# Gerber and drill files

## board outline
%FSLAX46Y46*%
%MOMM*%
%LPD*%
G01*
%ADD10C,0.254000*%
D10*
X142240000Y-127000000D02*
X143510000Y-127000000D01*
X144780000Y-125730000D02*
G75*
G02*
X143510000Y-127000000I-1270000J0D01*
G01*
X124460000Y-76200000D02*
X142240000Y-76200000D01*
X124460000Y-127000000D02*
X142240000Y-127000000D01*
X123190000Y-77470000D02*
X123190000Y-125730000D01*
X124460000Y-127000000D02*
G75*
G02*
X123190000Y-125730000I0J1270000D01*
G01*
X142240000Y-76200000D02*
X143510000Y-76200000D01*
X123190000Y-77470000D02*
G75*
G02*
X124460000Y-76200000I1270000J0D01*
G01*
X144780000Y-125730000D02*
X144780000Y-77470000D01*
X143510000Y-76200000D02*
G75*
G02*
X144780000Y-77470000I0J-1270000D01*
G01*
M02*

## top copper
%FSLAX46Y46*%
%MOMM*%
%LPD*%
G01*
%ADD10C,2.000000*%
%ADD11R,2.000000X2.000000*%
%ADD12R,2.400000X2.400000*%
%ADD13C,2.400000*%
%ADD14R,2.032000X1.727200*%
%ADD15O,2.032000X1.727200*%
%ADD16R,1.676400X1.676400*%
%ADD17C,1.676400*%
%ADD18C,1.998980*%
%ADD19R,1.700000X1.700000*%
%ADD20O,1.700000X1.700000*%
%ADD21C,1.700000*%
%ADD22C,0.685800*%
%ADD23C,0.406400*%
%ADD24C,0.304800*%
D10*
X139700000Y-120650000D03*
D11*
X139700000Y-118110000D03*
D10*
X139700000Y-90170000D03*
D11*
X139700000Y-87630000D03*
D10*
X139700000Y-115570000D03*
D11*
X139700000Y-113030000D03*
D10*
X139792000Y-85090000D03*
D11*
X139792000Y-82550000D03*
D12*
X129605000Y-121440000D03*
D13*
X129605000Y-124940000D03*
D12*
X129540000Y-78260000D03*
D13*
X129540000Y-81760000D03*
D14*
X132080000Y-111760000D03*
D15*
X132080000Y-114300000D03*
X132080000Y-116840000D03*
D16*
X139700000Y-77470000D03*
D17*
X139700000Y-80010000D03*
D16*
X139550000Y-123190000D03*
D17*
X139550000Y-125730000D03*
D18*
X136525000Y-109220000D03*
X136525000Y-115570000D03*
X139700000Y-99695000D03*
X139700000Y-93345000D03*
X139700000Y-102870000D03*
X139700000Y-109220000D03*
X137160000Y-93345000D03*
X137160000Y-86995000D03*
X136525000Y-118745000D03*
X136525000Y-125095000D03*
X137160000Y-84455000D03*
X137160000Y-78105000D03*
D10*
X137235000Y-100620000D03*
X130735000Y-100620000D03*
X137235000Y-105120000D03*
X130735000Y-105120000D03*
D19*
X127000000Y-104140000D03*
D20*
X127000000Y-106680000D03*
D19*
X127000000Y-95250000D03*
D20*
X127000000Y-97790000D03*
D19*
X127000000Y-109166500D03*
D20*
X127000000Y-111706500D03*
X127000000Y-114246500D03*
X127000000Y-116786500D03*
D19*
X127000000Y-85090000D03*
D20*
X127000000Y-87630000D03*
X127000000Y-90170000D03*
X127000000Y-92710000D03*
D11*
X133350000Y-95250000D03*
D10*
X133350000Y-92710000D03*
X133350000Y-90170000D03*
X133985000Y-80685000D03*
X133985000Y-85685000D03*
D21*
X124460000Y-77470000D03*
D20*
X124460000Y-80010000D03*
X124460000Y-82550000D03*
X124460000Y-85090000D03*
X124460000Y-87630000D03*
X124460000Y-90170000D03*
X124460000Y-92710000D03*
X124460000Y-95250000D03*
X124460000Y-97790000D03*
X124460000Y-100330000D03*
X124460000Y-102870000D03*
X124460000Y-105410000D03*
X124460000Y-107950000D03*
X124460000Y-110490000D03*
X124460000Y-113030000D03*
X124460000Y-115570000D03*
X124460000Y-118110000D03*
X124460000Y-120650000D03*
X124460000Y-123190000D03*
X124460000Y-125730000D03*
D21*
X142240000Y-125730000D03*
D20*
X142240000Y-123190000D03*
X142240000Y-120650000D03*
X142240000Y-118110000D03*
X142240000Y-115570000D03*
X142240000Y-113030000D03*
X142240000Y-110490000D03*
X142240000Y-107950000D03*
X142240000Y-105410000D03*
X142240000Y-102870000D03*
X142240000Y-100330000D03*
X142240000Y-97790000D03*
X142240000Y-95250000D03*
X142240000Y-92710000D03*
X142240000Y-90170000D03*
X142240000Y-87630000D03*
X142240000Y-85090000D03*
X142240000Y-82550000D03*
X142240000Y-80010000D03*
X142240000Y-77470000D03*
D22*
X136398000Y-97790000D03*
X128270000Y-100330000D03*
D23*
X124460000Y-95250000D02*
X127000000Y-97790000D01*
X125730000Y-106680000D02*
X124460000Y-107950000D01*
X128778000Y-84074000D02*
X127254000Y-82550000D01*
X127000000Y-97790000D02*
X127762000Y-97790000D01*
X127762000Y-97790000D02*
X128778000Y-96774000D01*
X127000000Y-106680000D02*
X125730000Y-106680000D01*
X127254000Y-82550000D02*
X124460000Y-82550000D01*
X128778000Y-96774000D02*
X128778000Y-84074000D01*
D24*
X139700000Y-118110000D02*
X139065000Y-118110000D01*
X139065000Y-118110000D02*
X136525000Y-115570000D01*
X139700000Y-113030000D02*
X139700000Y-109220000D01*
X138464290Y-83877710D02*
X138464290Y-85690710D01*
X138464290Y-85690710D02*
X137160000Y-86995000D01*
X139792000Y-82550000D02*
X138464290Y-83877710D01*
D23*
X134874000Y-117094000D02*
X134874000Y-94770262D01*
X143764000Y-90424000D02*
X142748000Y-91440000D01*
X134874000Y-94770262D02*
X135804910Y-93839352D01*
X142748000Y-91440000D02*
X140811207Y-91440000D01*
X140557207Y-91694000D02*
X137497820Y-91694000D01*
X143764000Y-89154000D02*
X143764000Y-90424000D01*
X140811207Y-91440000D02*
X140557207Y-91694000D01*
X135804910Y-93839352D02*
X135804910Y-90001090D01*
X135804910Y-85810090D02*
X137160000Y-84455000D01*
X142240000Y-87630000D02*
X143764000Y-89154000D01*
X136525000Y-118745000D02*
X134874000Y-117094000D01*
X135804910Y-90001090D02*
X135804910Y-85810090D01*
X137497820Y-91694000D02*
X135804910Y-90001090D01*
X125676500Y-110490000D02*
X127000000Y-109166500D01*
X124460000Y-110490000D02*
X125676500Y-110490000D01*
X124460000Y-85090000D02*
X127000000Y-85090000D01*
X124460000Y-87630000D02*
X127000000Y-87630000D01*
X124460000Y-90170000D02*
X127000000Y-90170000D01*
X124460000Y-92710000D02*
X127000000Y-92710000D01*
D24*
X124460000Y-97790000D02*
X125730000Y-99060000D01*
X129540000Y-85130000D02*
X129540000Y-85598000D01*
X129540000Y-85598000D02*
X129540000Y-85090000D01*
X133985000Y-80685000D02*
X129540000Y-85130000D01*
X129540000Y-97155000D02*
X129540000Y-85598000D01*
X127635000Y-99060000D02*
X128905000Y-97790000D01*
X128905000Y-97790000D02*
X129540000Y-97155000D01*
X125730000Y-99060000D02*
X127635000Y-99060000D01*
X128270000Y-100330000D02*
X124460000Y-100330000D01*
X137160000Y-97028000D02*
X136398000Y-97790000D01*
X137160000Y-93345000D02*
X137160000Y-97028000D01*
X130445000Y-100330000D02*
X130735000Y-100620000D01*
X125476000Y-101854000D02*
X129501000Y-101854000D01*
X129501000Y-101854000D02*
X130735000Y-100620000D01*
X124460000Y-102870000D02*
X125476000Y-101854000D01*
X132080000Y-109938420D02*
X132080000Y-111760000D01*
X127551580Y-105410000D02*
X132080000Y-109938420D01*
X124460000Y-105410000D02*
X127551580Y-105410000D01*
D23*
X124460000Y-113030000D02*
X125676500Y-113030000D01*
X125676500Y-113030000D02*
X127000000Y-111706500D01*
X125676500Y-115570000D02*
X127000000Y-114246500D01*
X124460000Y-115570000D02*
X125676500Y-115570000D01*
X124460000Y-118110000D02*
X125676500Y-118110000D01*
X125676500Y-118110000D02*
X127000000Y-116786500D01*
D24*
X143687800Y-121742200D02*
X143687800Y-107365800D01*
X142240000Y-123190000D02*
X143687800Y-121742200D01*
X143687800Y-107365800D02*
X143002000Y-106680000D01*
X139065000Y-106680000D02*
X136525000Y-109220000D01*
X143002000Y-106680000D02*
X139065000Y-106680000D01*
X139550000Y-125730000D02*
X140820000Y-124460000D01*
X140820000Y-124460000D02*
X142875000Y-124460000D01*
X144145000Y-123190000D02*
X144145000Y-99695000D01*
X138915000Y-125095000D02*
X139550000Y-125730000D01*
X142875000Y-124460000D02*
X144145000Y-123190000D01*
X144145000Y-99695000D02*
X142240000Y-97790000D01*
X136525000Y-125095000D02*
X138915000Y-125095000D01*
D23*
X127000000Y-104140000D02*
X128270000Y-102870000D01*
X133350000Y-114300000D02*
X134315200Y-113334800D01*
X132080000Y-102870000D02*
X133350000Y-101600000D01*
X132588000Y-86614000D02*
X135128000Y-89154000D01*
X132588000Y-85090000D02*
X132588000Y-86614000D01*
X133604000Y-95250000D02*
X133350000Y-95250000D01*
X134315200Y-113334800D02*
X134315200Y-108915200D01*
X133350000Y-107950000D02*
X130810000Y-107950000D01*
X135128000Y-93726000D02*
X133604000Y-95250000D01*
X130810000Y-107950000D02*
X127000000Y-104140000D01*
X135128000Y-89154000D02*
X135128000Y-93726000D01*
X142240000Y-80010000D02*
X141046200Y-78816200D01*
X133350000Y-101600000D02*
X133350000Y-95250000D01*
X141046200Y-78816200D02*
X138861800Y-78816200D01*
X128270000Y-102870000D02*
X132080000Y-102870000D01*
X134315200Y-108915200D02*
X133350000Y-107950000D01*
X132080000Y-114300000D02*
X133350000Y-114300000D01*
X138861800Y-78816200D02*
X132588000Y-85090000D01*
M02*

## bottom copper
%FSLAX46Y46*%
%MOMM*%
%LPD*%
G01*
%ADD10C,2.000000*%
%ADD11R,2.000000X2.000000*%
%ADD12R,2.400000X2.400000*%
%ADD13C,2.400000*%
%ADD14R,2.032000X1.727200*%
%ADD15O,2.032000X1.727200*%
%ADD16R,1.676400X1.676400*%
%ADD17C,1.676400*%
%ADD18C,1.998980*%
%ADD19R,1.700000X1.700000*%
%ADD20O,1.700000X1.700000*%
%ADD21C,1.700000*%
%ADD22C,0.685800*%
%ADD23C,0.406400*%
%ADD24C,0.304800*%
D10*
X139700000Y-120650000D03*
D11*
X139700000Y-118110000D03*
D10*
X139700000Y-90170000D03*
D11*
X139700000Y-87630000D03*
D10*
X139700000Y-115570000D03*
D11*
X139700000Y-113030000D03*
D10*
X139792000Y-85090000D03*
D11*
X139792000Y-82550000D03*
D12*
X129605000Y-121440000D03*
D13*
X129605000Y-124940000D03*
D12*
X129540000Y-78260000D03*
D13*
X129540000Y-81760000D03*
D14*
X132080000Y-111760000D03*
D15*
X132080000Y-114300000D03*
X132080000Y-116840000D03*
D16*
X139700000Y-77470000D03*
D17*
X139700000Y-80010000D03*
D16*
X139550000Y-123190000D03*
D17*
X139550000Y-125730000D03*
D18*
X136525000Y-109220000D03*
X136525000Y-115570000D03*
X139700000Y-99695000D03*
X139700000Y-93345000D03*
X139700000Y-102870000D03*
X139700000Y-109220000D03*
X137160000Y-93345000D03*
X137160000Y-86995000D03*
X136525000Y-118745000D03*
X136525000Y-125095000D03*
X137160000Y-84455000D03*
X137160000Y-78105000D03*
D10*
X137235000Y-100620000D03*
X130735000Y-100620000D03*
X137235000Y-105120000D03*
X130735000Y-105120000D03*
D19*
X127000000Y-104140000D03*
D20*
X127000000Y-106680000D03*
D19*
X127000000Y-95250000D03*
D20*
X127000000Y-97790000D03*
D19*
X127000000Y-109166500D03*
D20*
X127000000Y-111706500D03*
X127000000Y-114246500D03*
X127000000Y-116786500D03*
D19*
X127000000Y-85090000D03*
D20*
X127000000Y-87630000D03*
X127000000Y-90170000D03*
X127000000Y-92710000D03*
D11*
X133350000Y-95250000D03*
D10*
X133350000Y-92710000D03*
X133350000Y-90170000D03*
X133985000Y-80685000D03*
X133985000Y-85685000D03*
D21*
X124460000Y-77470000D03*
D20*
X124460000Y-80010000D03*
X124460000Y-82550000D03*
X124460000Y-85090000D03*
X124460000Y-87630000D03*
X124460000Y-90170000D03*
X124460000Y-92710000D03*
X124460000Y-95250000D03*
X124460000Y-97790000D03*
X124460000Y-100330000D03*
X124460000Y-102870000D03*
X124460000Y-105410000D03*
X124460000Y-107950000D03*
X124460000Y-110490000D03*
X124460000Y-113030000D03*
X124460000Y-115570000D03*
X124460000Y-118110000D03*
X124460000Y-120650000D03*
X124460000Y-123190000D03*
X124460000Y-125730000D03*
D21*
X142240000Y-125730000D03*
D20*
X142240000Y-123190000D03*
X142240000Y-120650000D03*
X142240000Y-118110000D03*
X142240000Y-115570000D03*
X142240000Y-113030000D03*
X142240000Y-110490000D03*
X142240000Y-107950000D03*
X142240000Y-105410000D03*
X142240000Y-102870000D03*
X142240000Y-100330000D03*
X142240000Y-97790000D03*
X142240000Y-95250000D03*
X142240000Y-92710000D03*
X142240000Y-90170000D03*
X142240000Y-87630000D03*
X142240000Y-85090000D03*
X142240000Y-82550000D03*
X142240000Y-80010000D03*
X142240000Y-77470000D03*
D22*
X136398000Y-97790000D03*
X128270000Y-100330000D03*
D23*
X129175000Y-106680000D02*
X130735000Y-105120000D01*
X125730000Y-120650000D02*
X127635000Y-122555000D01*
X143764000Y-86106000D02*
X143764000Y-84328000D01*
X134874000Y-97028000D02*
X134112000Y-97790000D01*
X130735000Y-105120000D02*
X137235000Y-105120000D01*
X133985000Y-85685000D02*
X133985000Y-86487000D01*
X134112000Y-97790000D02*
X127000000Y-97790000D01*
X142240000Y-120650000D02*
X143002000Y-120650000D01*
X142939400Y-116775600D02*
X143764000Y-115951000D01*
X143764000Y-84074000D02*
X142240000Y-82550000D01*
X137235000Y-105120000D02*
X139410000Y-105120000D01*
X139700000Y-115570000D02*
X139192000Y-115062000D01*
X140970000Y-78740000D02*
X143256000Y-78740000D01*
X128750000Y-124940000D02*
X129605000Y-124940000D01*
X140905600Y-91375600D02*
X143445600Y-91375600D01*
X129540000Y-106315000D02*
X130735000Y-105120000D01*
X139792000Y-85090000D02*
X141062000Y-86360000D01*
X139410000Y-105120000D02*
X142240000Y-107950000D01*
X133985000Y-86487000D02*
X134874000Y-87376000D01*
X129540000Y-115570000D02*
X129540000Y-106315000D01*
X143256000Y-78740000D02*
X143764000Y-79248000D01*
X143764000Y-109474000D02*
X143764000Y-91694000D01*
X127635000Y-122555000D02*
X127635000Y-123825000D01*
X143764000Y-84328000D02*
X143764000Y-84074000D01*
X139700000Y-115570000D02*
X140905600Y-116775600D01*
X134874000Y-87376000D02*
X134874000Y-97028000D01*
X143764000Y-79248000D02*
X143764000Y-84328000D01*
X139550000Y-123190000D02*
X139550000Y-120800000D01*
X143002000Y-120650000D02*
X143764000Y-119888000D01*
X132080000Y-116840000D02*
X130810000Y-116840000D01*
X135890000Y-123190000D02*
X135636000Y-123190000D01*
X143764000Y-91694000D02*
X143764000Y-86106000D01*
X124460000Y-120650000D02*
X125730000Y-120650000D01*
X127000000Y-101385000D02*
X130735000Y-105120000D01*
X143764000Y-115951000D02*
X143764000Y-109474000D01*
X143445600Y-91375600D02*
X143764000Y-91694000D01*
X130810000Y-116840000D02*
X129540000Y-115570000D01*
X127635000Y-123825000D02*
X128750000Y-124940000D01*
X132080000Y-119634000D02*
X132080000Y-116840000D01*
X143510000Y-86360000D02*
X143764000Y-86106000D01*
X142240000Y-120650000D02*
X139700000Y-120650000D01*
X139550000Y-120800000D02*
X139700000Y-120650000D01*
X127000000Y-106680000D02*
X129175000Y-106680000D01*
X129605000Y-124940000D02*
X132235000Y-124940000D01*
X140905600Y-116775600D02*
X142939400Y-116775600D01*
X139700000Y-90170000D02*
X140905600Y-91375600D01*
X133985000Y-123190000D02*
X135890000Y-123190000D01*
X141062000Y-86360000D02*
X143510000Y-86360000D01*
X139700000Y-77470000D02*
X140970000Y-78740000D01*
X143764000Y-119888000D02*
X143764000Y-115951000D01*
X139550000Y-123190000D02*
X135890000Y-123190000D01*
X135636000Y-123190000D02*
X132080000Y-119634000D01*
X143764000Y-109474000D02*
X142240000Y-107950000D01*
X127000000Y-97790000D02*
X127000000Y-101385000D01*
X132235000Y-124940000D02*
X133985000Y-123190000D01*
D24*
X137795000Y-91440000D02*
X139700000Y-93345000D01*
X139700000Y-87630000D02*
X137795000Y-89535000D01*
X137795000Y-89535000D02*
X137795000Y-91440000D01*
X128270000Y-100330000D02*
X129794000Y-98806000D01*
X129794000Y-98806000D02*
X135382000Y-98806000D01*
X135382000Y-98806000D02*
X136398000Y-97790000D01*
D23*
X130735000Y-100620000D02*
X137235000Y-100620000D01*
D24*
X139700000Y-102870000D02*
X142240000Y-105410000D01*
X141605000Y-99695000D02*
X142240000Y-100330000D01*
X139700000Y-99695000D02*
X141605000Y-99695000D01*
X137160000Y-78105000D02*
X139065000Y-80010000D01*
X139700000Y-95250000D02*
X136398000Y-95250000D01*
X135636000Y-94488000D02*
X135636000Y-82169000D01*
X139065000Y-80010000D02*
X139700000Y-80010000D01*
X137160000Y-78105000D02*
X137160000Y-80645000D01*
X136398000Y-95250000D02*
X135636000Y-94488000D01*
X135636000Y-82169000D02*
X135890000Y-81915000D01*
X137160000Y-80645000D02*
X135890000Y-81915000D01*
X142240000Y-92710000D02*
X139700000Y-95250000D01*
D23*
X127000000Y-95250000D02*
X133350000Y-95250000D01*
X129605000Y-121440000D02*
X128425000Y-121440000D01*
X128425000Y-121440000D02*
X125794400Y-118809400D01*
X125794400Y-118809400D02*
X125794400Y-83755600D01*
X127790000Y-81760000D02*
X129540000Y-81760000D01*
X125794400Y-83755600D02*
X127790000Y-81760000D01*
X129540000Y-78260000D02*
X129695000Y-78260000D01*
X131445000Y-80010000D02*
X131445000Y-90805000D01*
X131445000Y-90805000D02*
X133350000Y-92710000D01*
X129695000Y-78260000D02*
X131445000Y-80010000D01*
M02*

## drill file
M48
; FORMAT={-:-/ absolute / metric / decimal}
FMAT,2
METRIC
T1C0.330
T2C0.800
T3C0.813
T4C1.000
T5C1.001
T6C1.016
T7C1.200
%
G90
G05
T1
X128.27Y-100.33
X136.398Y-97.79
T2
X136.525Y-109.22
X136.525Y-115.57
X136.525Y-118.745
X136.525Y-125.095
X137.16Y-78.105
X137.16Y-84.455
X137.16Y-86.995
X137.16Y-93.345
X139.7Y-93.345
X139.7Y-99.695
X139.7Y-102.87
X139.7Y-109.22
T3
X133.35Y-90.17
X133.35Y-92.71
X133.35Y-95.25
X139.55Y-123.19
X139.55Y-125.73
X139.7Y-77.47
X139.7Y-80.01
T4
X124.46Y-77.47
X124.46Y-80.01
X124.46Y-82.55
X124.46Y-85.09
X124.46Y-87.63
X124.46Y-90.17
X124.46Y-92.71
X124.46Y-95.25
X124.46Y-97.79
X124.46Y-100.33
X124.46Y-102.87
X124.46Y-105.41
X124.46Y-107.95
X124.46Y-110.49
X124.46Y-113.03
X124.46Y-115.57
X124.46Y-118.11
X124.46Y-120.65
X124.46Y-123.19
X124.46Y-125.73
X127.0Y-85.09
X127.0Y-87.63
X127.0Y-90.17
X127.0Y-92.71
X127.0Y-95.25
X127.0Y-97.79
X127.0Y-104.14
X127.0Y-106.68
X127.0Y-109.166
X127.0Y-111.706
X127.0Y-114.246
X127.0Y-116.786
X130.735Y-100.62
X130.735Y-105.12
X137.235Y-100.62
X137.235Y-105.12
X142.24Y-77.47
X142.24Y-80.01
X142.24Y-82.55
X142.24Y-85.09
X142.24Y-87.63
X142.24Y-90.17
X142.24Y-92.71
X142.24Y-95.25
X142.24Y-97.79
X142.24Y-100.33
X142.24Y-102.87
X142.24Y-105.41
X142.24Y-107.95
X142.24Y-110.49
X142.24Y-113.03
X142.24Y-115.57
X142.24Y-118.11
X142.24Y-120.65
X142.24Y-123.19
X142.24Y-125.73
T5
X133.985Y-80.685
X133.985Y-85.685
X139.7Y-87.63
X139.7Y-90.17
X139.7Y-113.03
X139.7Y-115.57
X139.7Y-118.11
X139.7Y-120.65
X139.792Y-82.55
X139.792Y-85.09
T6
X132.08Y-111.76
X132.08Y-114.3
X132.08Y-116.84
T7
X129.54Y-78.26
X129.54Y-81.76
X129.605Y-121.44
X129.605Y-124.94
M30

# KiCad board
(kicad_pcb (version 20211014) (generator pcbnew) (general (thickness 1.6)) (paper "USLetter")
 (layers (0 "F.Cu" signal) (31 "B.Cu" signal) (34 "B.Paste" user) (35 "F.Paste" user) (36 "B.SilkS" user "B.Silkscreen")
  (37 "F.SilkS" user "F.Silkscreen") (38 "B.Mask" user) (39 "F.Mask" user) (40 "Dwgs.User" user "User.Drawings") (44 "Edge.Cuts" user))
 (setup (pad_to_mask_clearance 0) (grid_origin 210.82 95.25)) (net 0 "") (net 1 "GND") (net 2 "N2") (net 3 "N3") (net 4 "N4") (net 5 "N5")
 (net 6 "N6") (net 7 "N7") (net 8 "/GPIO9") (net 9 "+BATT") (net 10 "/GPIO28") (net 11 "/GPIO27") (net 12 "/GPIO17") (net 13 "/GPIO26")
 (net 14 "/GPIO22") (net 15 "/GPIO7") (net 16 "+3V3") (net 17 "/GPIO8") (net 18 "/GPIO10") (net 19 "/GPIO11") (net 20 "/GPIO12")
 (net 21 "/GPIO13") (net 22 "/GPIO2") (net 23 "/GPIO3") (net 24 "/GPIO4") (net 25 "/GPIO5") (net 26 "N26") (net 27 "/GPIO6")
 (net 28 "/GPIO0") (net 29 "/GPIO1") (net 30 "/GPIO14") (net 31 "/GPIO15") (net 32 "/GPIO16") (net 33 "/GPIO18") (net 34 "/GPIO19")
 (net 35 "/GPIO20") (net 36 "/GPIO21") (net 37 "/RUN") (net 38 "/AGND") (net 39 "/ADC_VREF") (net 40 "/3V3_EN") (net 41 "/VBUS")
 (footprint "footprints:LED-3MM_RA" (layer "F.Cu") (at 139.7 120.65 90)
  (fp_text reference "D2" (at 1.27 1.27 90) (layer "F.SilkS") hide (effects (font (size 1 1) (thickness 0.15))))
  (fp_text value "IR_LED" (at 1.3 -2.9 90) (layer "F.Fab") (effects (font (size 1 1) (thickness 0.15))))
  (pad "1" thru_hole circle locked (at 0 0 180) (size 2 2) (drill 1.00076) (layers *.Cu *.Mask "F.SilkS") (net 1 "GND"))
  (pad "2" thru_hole rect locked (at 2.54 0 90) (size 2 2) (drill 1.00076) (layers *.Cu *.Mask "F.SilkS") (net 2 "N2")))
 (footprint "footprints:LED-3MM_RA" (layer "F.Cu") (at 139.7 90.17 90)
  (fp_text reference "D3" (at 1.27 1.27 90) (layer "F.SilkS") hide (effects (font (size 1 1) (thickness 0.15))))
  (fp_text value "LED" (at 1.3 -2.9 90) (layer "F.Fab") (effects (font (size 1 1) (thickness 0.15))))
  (pad "1" thru_hole circle locked (at 0 0 180) (size 2 2) (drill 1.00076) (layers *.Cu *.Mask "F.SilkS") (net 1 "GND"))
  (pad "2" thru_hole rect locked (at 2.54 0 90) (size 2 2) (drill 1.00076) (layers *.Cu *.Mask "F.SilkS") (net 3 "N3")))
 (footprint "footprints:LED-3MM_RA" (layer "F.Cu") (at 139.7 115.57 90)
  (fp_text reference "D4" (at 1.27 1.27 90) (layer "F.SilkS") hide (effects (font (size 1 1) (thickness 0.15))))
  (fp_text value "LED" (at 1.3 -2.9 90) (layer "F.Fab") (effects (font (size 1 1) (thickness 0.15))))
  (pad "1" thru_hole circle locked (at 0 0 180) (size 2 2) (drill 1.00076) (layers *.Cu *.Mask "F.SilkS") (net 1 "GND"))
  (pad "2" thru_hole rect locked (at 2.54 0 90) (size 2 2) (drill 1.00076) (layers *.Cu *.Mask "F.SilkS") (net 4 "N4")))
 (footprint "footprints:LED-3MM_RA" (layer "F.Cu") (at 139.792 85.09 90)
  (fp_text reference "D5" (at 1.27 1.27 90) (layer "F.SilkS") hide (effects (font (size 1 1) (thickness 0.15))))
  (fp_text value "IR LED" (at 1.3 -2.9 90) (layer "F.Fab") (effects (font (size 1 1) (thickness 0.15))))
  (pad "1" thru_hole circle locked (at 0 0 180) (size 2 2) (drill 1.00076) (layers *.Cu *.Mask "F.SilkS") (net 1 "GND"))
  (pad "2" thru_hole rect locked (at 2.54 0 90) (size 2 2) (drill 1.00076) (layers *.Cu *.Mask "F.SilkS") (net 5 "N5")))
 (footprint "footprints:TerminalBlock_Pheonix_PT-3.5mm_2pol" (layer "F.Cu") (at 129.605 121.44 -90)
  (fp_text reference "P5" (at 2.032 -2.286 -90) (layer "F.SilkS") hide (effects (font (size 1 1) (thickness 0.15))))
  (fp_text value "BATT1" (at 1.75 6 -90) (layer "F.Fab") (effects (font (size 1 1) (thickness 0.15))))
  (pad "1" thru_hole rect locked (at 0 0 270) (size 2.4 2.4) (drill 1.2) (layers *.Cu *.Mask "F.SilkS") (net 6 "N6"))
  (pad "2" thru_hole circle locked (at 3.5 0 270) (size 2.4 2.4) (drill 1.2) (layers *.Cu *.Mask "F.SilkS") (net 1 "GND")))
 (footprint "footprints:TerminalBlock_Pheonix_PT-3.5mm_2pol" (layer "F.Cu") (at 129.54 78.26 -90)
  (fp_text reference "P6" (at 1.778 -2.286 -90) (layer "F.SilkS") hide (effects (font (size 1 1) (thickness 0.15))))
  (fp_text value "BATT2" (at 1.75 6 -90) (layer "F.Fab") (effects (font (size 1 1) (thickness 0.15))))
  (pad "1" thru_hole rect (at 0 0 270) (size 2.4 2.4) (drill 1.2) (layers *.Cu *.Mask "F.SilkS") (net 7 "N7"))
  (pad "2" thru_hole circle (at 3.5 0 270) (size 2.4 2.4) (drill 1.2) (layers *.Cu *.Mask "F.SilkS") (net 6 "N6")))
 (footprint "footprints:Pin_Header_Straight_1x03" (layer "F.Cu") (at 132.08 111.76)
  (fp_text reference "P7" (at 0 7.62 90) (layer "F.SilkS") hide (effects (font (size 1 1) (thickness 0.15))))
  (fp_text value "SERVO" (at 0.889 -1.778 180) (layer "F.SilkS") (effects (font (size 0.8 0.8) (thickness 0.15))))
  (pad "1" thru_hole rect (at 0 0) (size 2.032 1.7272) (drill 1.016) (layers *.Cu *.Mask "F.SilkS") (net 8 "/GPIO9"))
  (pad "2" thru_hole oval (at 0 2.54) (size 2.032 1.7272) (drill 1.016) (layers *.Cu *.Mask "F.SilkS") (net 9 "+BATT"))
  (pad "3" thru_hole oval (at 0 5.08) (size 2.032 1.7272) (drill 1.016) (layers *.Cu *.Mask "F.SilkS") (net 1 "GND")))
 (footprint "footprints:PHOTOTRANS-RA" (layer "F.Cu") (at 139.7 78.74 90)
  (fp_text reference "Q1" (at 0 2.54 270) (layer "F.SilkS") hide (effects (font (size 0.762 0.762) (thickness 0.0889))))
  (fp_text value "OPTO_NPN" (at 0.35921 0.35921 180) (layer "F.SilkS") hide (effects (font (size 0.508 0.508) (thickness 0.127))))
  (pad "1" thru_hole rect locked (at 1.27 0 90) (size 1.6764 1.6764) (drill 0.8128) (layers *.Cu *.Mask "F.SilkS") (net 1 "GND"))
  (pad "3" thru_hole circle locked (at -1.27 0 90) (size 1.6764 1.6764) (drill 0.8128) (layers *.Cu *.Mask "F.SilkS") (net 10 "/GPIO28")))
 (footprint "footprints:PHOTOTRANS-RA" (layer "F.Cu") (at 139.55 124.46 90)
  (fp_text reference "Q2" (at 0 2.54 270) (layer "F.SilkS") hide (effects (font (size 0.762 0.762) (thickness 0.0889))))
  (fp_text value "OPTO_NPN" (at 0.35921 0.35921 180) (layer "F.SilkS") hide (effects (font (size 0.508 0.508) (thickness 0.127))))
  (pad "1" thru_hole rect locked (at 1.27 0 90) (size 1.6764 1.6764) (drill 0.8128) (layers *.Cu *.Mask "F.SilkS") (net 1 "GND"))
  (pad "3" thru_hole circle locked (at -1.27 0 90) (size 1.6764 1.6764) (drill 0.8128) (layers *.Cu *.Mask "F.SilkS") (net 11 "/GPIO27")))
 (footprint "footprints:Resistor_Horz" (layer "F.Cu") (at 136.525 112.395 -90)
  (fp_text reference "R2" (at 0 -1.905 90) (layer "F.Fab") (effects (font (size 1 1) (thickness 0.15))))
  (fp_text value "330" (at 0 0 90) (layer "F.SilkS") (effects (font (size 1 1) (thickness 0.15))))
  (pad "1" thru_hole circle locked (at -3.175 0 270) (size 1.99898 1.99898) (drill 0.8) (layers *.Cu *.SilkS *.Mask) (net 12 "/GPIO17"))
  (pad "2" thru_hole circle locked (at 3.175 0 270) (size 1.99898 1.99898) (drill 0.8) (layers *.Cu *.SilkS *.Mask) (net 2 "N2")))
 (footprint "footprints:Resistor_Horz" (layer "F.Cu") (at 139.7 96.52 90)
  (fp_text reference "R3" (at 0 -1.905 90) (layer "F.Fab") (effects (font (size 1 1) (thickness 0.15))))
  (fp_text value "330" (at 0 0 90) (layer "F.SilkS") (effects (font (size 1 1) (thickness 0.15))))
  (pad "1" thru_hole circle locked (at -3.175 0 90) (size 1.99898 1.99898) (drill 0.8) (layers *.Cu *.SilkS *.Mask) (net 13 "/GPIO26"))
  (pad "2" thru_hole circle locked (at 3.175 0 90) (size 1.99898 1.99898) (drill 0.8) (layers *.Cu *.SilkS *.Mask) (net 3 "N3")))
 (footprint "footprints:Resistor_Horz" (layer "F.Cu") (at 139.7 106.045 -90)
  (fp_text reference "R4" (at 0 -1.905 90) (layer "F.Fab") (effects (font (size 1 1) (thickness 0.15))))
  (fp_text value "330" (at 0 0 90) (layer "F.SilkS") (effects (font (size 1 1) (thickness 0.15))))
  (pad "1" thru_hole circle locked (at -3.175 0 270) (size 1.99898 1.99898) (drill 0.8) (layers *.Cu *.SilkS *.Mask) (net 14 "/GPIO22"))
  (pad "2" thru_hole circle locked (at 3.175 0 270) (size 1.99898 1.99898) (drill 0.8) (layers *.Cu *.SilkS *.Mask) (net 4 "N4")))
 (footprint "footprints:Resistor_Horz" (layer "F.Cu") (at 137.16 90.17 90)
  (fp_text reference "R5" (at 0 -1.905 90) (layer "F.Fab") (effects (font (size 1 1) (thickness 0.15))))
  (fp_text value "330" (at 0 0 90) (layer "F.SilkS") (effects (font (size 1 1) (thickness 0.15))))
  (pad "1" thru_hole circle locked (at -3.175 0 90) (size 1.99898 1.99898) (drill 0.8) (layers *.Cu *.SilkS *.Mask) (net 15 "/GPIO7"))
  (pad "2" thru_hole circle locked (at 3.175 0 90) (size 1.99898 1.99898) (drill 0.8) (layers *.Cu *.SilkS *.Mask) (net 5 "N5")))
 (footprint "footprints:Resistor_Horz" (layer "F.Cu") (at 136.525 121.92 -90)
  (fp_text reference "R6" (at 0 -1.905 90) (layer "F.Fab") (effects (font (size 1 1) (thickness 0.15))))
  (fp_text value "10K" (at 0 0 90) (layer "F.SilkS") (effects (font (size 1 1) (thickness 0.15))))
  (pad "1" thru_hole circle locked (at -3.175 0 270) (size 1.99898 1.99898) (drill 0.8) (layers *.Cu *.SilkS *.Mask) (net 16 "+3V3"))
  (pad "2" thru_hole circle locked (at 3.175 0 270) (size 1.99898 1.99898) (drill 0.8) (layers *.Cu *.SilkS *.Mask) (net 11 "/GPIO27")))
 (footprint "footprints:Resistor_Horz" (layer "F.Cu") (at 137.16 81.28 90)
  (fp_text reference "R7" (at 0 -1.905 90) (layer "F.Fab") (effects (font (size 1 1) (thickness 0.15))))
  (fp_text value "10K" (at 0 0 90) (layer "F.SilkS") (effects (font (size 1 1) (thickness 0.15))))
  (pad "1" thru_hole circle locked (at -3.175 0 90) (size 1.99898 1.99898) (drill 0.8) (layers *.Cu *.SilkS *.Mask) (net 16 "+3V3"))
  (pad "2" thru_hole circle locked (at 3.175 0 90) (size 1.99898 1.99898) (drill 0.8) (layers *.Cu *.SilkS *.Mask) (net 10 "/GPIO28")))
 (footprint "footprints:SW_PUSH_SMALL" (layer "F.Cu") (at 133.985 102.87)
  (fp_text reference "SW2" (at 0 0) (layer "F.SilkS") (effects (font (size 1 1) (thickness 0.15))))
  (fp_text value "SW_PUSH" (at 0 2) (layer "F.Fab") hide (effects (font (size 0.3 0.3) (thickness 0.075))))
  (pad "1" thru_hole circle locked (at 3.25 -2.25) (size 2 2) (drill 1) (layers *.Cu *.Mask "F.SilkS") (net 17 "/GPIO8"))
  (pad "1" thru_hole circle locked (at -3.25 -2.25) (size 2 2) (drill 1) (layers *.Cu *.Mask "F.SilkS") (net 17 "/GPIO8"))
  (pad "2" thru_hole circle locked (at 3.25 2.25) (size 2 2) (drill 1) (layers *.Cu *.Mask "F.SilkS") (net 1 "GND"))
  (pad "2" thru_hole circle locked (at -3.25 2.25) (size 2 2) (drill 1) (layers *.Cu *.Mask "F.SilkS") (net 1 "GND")))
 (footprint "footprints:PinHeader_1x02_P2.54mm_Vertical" (layer "F.Cu") (at 127 104.14)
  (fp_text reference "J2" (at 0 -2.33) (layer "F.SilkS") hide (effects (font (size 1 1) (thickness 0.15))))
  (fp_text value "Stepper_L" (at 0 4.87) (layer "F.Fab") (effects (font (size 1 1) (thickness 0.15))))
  (pad "1" thru_hole rect (at 0 0) (size 1.7 1.7) (drill 1) (layers *.Cu *.Mask) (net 9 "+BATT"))
  (pad "2" thru_hole oval (at 0 2.54) (size 1.7 1.7) (drill 1) (layers *.Cu *.Mask) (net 1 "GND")))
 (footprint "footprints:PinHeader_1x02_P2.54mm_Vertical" (layer "F.Cu") (at 127 95.25)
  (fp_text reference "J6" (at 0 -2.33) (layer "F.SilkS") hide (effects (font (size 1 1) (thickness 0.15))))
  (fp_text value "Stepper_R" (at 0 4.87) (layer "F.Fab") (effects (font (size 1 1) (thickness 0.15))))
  (pad "1" thru_hole rect (at 0 0) (size 1.7 1.7) (drill 1) (layers *.Cu *.Mask) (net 9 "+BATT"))
  (pad "2" thru_hole oval (at 0 2.54) (size 1.7 1.7) (drill 1) (layers *.Cu *.Mask) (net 1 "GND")))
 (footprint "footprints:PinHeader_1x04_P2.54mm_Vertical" (layer "F.Cu") (at 127 109.1665)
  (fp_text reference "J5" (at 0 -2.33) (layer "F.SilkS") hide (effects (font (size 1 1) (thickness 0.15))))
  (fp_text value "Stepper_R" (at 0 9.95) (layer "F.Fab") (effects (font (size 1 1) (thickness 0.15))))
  (pad "1" thru_hole rect (at 0 0) (size 1.7 1.7) (drill 1) (layers *.Cu *.Mask) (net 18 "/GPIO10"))
  (pad "2" thru_hole oval (at 0 2.54) (size 1.7 1.7) (drill 1) (layers *.Cu *.Mask) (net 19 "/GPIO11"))
  (pad "3" thru_hole oval (at 0 5.08) (size 1.7 1.7) (drill 1) (layers *.Cu *.Mask) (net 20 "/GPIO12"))
  (pad "4" thru_hole oval (at 0 7.62) (size 1.7 1.7) (drill 1) (layers *.Cu *.Mask) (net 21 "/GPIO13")))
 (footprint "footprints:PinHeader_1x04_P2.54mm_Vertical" (layer "F.Cu") (at 127 85.09)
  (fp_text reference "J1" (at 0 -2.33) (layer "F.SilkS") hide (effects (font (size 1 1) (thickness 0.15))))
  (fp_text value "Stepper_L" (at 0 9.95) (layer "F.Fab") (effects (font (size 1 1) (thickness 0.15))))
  (pad "1" thru_hole rect (at 0 0) (size 1.7 1.7) (drill 1) (layers *.Cu *.Mask) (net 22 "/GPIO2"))
  (pad "2" thru_hole oval (at 0 2.54) (size 1.7 1.7) (drill 1) (layers *.Cu *.Mask) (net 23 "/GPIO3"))
  (pad "3" thru_hole oval (at 0 5.08) (size 1.7 1.7) (drill 1) (layers *.Cu *.Mask) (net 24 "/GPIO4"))
  (pad "4" thru_hole oval (at 0 7.62) (size 1.7 1.7) (drill 1) (layers *.Cu *.Mask) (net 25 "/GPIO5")))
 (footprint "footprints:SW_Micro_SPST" (layer "F.Cu") (at 133.35 92.71 90)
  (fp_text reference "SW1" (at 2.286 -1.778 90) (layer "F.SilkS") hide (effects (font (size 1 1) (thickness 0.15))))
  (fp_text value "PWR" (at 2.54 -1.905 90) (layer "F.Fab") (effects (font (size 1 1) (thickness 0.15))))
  (pad "1" thru_hole rect (at -2.54 0 90) (size 2 2) (drill 0.8128) (layers *.Cu *.Mask "F.SilkS") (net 9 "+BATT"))
  (pad "2" thru_hole circle (at 0 0 90) (size 2 2) (drill 0.8128) (layers *.Cu *.Mask "F.SilkS") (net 7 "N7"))
  (pad "3" thru_hole circle (at 2.54 0 90) (size 2 2) (drill 0.8128) (layers *.Cu *.Mask "F.SilkS") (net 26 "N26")))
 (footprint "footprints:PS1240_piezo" (layer "B.Cu") (at 133.985 83.185 -90)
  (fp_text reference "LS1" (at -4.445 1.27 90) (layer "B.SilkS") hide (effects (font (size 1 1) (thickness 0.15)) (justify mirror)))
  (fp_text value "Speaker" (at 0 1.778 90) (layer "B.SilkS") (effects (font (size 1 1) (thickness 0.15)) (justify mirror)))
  (pad "1" thru_hole circle (at -2.5 0 270) (size 2 2) (drill 1.00076) (layers *.Cu *.Mask "B.SilkS") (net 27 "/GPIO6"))
  (pad "2" thru_hole circle (at 2.5 0 270) (size 2 2) (drill 1.00076) (layers *.Cu *.Mask "B.SilkS") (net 1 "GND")))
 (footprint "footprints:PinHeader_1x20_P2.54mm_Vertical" (layer "B.Cu") (at 124.46 77.47 180)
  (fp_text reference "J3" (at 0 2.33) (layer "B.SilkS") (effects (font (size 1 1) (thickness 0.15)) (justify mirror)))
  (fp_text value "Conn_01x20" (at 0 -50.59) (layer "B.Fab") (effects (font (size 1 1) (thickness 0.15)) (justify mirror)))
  (pad "1" thru_hole circle (at 0 0) (size 1.7 1.7) (drill 1) (layers *.Cu *.Mask) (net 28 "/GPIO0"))
  (pad "2" thru_hole oval (at 0 -2.54) (size 1.7 1.7) (drill 1) (layers *.Cu *.Mask) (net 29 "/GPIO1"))
  (pad "3" thru_hole oval (at 0 -5.08) (size 1.7 1.7) (drill 1) (layers *.Cu *.Mask) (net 1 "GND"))
  (pad "4" thru_hole oval (at 0 -7.62) (size 1.7 1.7) (drill 1) (layers *.Cu *.Mask) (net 22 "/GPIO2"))
  (pad "5" thru_hole oval (at 0 -10.16) (size 1.7 1.7) (drill 1) (layers *.Cu *.Mask) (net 23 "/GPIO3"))
  (pad "6" thru_hole oval (at 0 -12.7) (size 1.7 1.7) (drill 1) (layers *.Cu *.Mask) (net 24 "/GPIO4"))
  (pad "7" thru_hole oval (at 0 -15.24) (size 1.7 1.7) (drill 1) (layers *.Cu *.Mask) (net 25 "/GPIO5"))
  (pad "8" thru_hole oval (at 0 -17.78) (size 1.7 1.7) (drill 1) (layers *.Cu *.Mask) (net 1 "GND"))
  (pad "9" thru_hole oval (at 0 -20.32) (size 1.7 1.7) (drill 1) (layers *.Cu *.Mask) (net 27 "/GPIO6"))
  (pad "10" thru_hole oval (at 0 -22.86) (size 1.7 1.7) (drill 1) (layers *.Cu *.Mask) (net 15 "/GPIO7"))
  (pad "11" thru_hole oval (at 0 -25.4) (size 1.7 1.7) (drill 1) (layers *.Cu *.Mask) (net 17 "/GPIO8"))
  (pad "12" thru_hole oval (at 0 -27.94) (size 1.7 1.7) (drill 1) (layers *.Cu *.Mask) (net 8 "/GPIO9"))
  (pad "13" thru_hole oval (at 0 -30.48) (size 1.7 1.7) (drill 1) (layers *.Cu *.Mask) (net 1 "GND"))
  (pad "14" thru_hole oval (at 0 -33.02) (size 1.7 1.7) (drill 1) (layers *.Cu *.Mask) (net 18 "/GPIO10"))
  (pad "15" thru_hole oval (at 0 -35.56) (size 1.7 1.7) (drill 1) (layers *.Cu *.Mask) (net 19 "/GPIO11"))
  (pad "16" thru_hole oval (at 0 -38.1) (size 1.7 1.7) (drill 1) (layers *.Cu *.Mask) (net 20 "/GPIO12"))
  (pad "17" thru_hole oval (at 0 -40.64) (size 1.7 1.7) (drill 1) (layers *.Cu *.Mask) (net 21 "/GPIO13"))
  (pad "18" thru_hole oval (at 0 -43.18) (size 1.7 1.7) (drill 1) (layers *.Cu *.Mask) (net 1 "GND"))
  (pad "19" thru_hole oval (at 0 -45.72) (size 1.7 1.7) (drill 1) (layers *.Cu *.Mask) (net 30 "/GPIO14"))
  (pad "20" thru_hole oval (at 0 -48.26) (size 1.7 1.7) (drill 1) (layers *.Cu *.Mask) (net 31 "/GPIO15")))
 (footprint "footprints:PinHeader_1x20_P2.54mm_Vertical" (layer "B.Cu") (at 142.24 125.73)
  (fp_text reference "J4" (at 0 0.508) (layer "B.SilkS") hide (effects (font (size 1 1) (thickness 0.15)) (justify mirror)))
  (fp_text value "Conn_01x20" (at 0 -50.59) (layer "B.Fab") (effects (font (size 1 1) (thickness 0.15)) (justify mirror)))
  (pad "1" thru_hole circle (at 0 0 180) (size 1.7 1.7) (drill 1) (layers *.Cu *.Mask) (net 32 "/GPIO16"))
  (pad "2" thru_hole oval (at 0 -2.54 180) (size 1.7 1.7) (drill 1) (layers *.Cu *.Mask) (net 12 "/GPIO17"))
  (pad "3" thru_hole oval (at 0 -5.08 180) (size 1.7 1.7) (drill 1) (layers *.Cu *.Mask) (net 1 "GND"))
  (pad "4" thru_hole oval (at 0 -7.62 180) (size 1.7 1.7) (drill 1) (layers *.Cu *.Mask) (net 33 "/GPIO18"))
  (pad "5" thru_hole oval (at 0 -10.16 180) (size 1.7 1.7) (drill 1) (layers *.Cu *.Mask) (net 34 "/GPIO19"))
  (pad "6" thru_hole oval (at 0 -12.7 180) (size 1.7 1.7) (drill 1) (layers *.Cu *.Mask) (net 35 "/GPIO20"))
  (pad "7" thru_hole oval (at 0 -15.24 180) (size 1.7 1.7) (drill 1) (layers *.Cu *.Mask) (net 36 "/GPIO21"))
  (pad "8" thru_hole oval (at 0 -17.78 180) (size 1.7 1.7) (drill 1) (layers *.Cu *.Mask) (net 1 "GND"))
  (pad "9" thru_hole oval (at 0 -20.32 180) (size 1.7 1.7) (drill 1) (layers *.Cu *.Mask) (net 14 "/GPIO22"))
  (pad "10" thru_hole oval (at 0 -22.86 180) (size 1.7 1.7) (drill 1) (layers *.Cu *.Mask) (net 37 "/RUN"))
  (pad "11" thru_hole oval (at 0 -25.4 180) (size 1.7 1.7) (drill 1) (layers *.Cu *.Mask) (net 13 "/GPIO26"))
  (pad "12" thru_hole oval (at 0 -27.94 180) (size 1.7 1.7) (drill 1) (layers *.Cu *.Mask) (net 11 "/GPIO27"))
  (pad "13" thru_hole oval (at 0 -30.48 180) (size 1.7 1.7) (drill 1) (layers *.Cu *.Mask) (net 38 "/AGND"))
  (pad "14" thru_hole oval (at 0 -33.02 180) (size 1.7 1.7) (drill 1) (layers *.Cu *.Mask) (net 10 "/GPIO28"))
  (pad "15" thru_hole oval (at 0 -35.56 180) (size 1.7 1.7) (drill 1) (layers *.Cu *.Mask) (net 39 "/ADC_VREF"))
  (pad "16" thru_hole oval (at 0 -38.1 180) (size 1.7 1.7) (drill 1) (layers *.Cu *.Mask) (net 16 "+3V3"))
  (pad "17" thru_hole oval (at 0 -40.64 180) (size 1.7 1.7) (drill 1) (layers *.Cu *.Mask) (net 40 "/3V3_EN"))
  (pad "18" thru_hole oval (at 0 -43.18 180) (size 1.7 1.7) (drill 1) (layers *.Cu *.Mask) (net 1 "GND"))
  (pad "19" thru_hole oval (at 0 -45.72 180) (size 1.7 1.7) (drill 1) (layers *.Cu *.Mask) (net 9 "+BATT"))
  (pad "20" thru_hole oval (at 0 -48.26 180) (size 1.7 1.7) (drill 1) (layers *.Cu *.Mask) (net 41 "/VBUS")))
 (gr_line (start 142.24 127) (end 143.51 127) (layer "Edge.Cuts") (width 0.254))
 (gr_arc (start 144.78 125.73) (mid 144.408026 126.628026) (end 143.51 127) (layer "Edge.Cuts") (width 0.254))
 (gr_line (start 124.46 76.2) (end 142.24 76.2) (layer "Edge.Cuts") (width 0.254))
 (gr_line (start 124.46 127) (end 142.24 127) (layer "Edge.Cuts") (width 0.254))
 (gr_line (start 123.19 77.47) (end 123.19 125.73) (layer "Edge.Cuts") (width 0.254))
 (gr_arc (start 124.46 127) (mid 123.561974 126.628026) (end 123.19 125.73) (layer "Edge.Cuts") (width 0.254))
 (gr_line (start 142.24 76.2) (end 143.51 76.2) (layer "Edge.Cuts") (width 0.254))
 (gr_arc (start 123.19 77.47) (mid 123.561974 76.571974) (end 124.46 76.2) (layer "Edge.Cuts") (width 0.254))
 (gr_line (start 144.78 125.73) (end 144.78 77.47) (layer "Edge.Cuts") (width 0.254))
 (gr_arc (start 143.51 76.2) (mid 144.408026 76.571974) (end 144.78 77.47) (layer "Edge.Cuts") (width 0.254))
 (segment (start 124.46 95.25) (end 127 97.79) (width 0.4064) (layer "F.Cu") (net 1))
 (segment (start 125.73 106.68) (end 124.46 107.95) (width 0.4064) (layer "F.Cu") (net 1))
 (segment (start 128.778 84.074) (end 127.254 82.55) (width 0.4064) (layer "F.Cu") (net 1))
 (segment (start 127 97.79) (end 127.762 97.79) (width 0.4064) (layer "F.Cu") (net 1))
 (segment (start 127.762 97.79) (end 128.778 96.774) (width 0.4064) (layer "F.Cu") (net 1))
 (segment (start 127 106.68) (end 125.73 106.68) (width 0.4064) (layer "F.Cu") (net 1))
 (segment (start 127.254 82.55) (end 124.46 82.55) (width 0.4064) (layer "F.Cu") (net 1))
 (segment (start 128.778 96.774) (end 128.778 84.074) (width 0.4064) (layer "F.Cu") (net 1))
 (segment (start 129.175 106.68) (end 130.735 105.12) (width 0.4064) (layer "B.Cu") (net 1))
 (segment (start 125.73 120.65) (end 127.635 122.555) (width 0.4064) (layer "B.Cu") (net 1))
 (segment (start 143.764 86.106) (end 143.764 84.328) (width 0.4064) (layer "B.Cu") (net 1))
 (segment (start 134.874 97.028) (end 134.112 97.79) (width 0.4064) (layer "B.Cu") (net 1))
 (segment (start 130.735 105.12) (end 137.235 105.12) (width 0.4064) (layer "B.Cu") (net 1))
 (segment (start 133.985 85.685) (end 133.985 86.487) (width 0.4064) (layer "B.Cu") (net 1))
 (segment (start 134.112 97.79) (end 127 97.79) (width 0.4064) (layer "B.Cu") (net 1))
 (segment (start 142.24 120.65) (end 143.002 120.65) (width 0.4064) (layer "B.Cu") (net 1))
 (segment (start 142.9394 116.7756) (end 143.764 115.951) (width 0.4064) (layer "B.Cu") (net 1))
 (segment (start 143.764 84.074) (end 142.24 82.55) (width 0.4064) (layer "B.Cu") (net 1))
 (segment (start 137.235 105.12) (end 139.41 105.12) (width 0.4064) (layer "B.Cu") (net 1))
 (segment (start 139.7 115.57) (end 139.192 115.062) (width 0.4064) (layer "B.Cu") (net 1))
 (segment (start 140.97 78.74) (end 143.256 78.74) (width 0.4064) (layer "B.Cu") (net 1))
 (segment (start 128.75 124.94) (end 129.605 124.94) (width 0.4064) (layer "B.Cu") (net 1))
 (segment (start 140.9056 91.3756) (end 143.4456 91.3756) (width 0.4064) (layer "B.Cu") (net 1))
 (segment (start 129.54 106.315) (end 130.735 105.12) (width 0.4064) (layer "B.Cu") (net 1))
 (segment (start 139.792 85.09) (end 141.062 86.36) (width 0.4064) (layer "B.Cu") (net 1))
 (segment (start 139.41 105.12) (end 142.24 107.95) (width 0.4064) (layer "B.Cu") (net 1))
 (segment (start 133.985 86.487) (end 134.874 87.376) (width 0.4064) (layer "B.Cu") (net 1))
 (segment (start 129.54 115.57) (end 129.54 106.315) (width 0.4064) (layer "B.Cu") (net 1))
 (segment (start 143.256 78.74) (end 143.764 79.248) (width 0.4064) (layer "B.Cu") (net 1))
 (segment (start 143.764 109.474) (end 143.764 91.694) (width 0.4064) (layer "B.Cu") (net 1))
 (segment (start 127.635 122.555) (end 127.635 123.825) (width 0.4064) (layer "B.Cu") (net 1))
 (segment (start 143.764 84.328) (end 143.764 84.074) (width 0.4064) (layer "B.Cu") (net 1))
 (segment (start 139.7 115.57) (end 140.9056 116.7756) (width 0.4064) (layer "B.Cu") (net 1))
 (segment (start 134.874 87.376) (end 134.874 97.028) (width 0.4064) (layer "B.Cu") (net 1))
 (segment (start 143.764 79.248) (end 143.764 84.328) (width 0.4064) (layer "B.Cu") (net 1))
 (segment (start 139.55 123.19) (end 139.55 120.8) (width 0.4064) (layer "B.Cu") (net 1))
 (segment (start 143.002 120.65) (end 143.764 119.888) (width 0.4064) (layer "B.Cu") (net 1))
 (segment (start 132.08 116.84) (end 130.81 116.84) (width 0.4064) (layer "B.Cu") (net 1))
 (segment (start 135.89 123.19) (end 135.636 123.19) (width 0.4064) (layer "B.Cu") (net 1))
 (segment (start 143.764 91.694) (end 143.764 86.106) (width 0.4064) (layer "B.Cu") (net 1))
 (segment (start 124.46 120.65) (end 125.73 120.65) (width 0.4064) (layer "B.Cu") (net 1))
 (segment (start 127 101.385) (end 130.735 105.12) (width 0.4064) (layer "B.Cu") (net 1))
 (segment (start 143.764 115.951) (end 143.764 109.474) (width 0.4064) (layer "B.Cu") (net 1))
 (segment (start 143.4456 91.3756) (end 143.764 91.694) (width 0.4064) (layer "B.Cu") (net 1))
 (segment (start 130.81 116.84) (end 129.54 115.57) (width 0.4064) (layer "B.Cu") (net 1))
 (segment (start 127.635 123.825) (end 128.75 124.94) (width 0.4064) (layer "B.Cu") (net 1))
 (segment (start 132.08 119.634) (end 132.08 116.84) (width 0.4064) (layer "B.Cu") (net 1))
 (segment (start 143.51 86.36) (end 143.764 86.106) (width 0.4064) (layer "B.Cu") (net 1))
 (segment (start 142.24 120.65) (end 139.7 120.65) (width 0.4064) (layer "B.Cu") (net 1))
 (segment (start 139.55 120.8) (end 139.7 120.65) (width 0.4064) (layer "B.Cu") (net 1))
 (segment (start 127 106.68) (end 129.175 106.68) (width 0.4064) (layer "B.Cu") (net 1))
 (segment (start 129.605 124.94) (end 132.235 124.94) (width 0.4064) (layer "B.Cu") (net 1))
 (segment (start 140.9056 116.7756) (end 142.9394 116.7756) (width 0.4064) (layer "B.Cu") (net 1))
 (segment (start 139.7 90.17) (end 140.9056 91.3756) (width 0.4064) (layer "B.Cu") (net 1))
 (segment (start 133.985 123.19) (end 135.89 123.19) (width 0.4064) (layer "B.Cu") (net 1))
 (segment (start 141.062 86.36) (end 143.51 86.36) (width 0.4064) (layer "B.Cu") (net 1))
 (segment (start 139.7 77.47) (end 140.97 78.74) (width 0.4064) (layer "B.Cu") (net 1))
 (segment (start 143.764 119.888) (end 143.764 115.951) (width 0.4064) (layer "B.Cu") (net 1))
 (segment (start 139.55 123.19) (end 135.89 123.19) (width 0.4064) (layer "B.Cu") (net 1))
 (segment (start 135.636 123.19) (end 132.08 119.634) (width 0.4064) (layer "B.Cu") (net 1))
 (segment (start 143.764 109.474) (end 142.24 107.95) (width 0.4064) (layer "B.Cu") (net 1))
 (segment (start 127 97.79) (end 127 101.385) (width 0.4064) (layer "B.Cu") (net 1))
 (segment (start 132.235 124.94) (end 133.985 123.19) (width 0.4064) (layer "B.Cu") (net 1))
 (segment (start 139.7 118.11) (end 139.065 118.11) (width 0.3048) (layer "F.Cu") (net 2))
 (segment (start 139.065 118.11) (end 136.525 115.57) (width 0.3048) (layer "F.Cu") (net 2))
 (segment (start 137.795 91.44) (end 139.7 93.345) (width 0.3048) (layer "B.Cu") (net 3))
 (segment (start 139.7 87.63) (end 137.795 89.535) (width 0.3048) (layer "B.Cu") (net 3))
 (segment (start 137.795 89.535) (end 137.795 91.44) (width 0.3048) (layer "B.Cu") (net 3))
 (segment (start 139.7 113.03) (end 139.7 109.22) (width 0.3048) (layer "F.Cu") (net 4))
 (segment (start 138.46429 83.87771) (end 138.46429 85.69071) (width 0.3048) (layer "F.Cu") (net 5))
 (segment (start 138.46429 85.69071) (end 137.16 86.995) (width 0.3048) (layer "F.Cu") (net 5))
 (segment (start 139.792 82.55) (end 138.46429 83.87771) (width 0.3048) (layer "F.Cu") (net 5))
 (segment (start 134.874 117.094) (end 134.874 94.770262) (width 0.4064) (layer "F.Cu") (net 16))
 (segment (start 143.764 90.424) (end 142.748 91.44) (width 0.4064) (layer "F.Cu") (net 16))
 (segment (start 134.874 94.770262) (end 135.80491 93.839352) (width 0.4064) (layer "F.Cu") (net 16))
 (segment (start 142.748 91.44) (end 140.811207 91.44) (width 0.4064) (layer "F.Cu") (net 16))
 (segment (start 140.557207 91.694) (end 137.49782 91.694) (width 0.4064) (layer "F.Cu") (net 16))
 (segment (start 143.764 89.154) (end 143.764 90.424) (width 0.4064) (layer "F.Cu") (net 16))
 (segment (start 140.811207 91.44) (end 140.557207 91.694) (width 0.4064) (layer "F.Cu") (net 16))
 (segment (start 135.80491 93.839352) (end 135.80491 90.00109) (width 0.4064) (layer "F.Cu") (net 16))
 (segment (start 135.80491 85.81009) (end 137.16 84.455) (width 0.4064) (layer "F.Cu") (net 16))
 (segment (start 142.24 87.63) (end 143.764 89.154) (width 0.4064) (layer "F.Cu") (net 16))
 (segment (start 136.525 118.745) (end 134.874 117.094) (width 0.4064) (layer "F.Cu") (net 16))
 (segment (start 135.80491 90.00109) (end 135.80491 85.81009) (width 0.4064) (layer "F.Cu") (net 16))
 (segment (start 137.49782 91.694) (end 135.80491 90.00109) (width 0.4064) (layer "F.Cu") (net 16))
 (segment (start 125.6765 110.49) (end 127 109.1665) (width 0.4064) (layer "F.Cu") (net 18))
 (segment (start 124.46 110.49) (end 125.6765 110.49) (width 0.4064) (layer "F.Cu") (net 18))
 (segment (start 124.46 85.09) (end 127 85.09) (width 0.4064) (layer "F.Cu") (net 22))
 (segment (start 124.46 87.63) (end 127 87.63) (width 0.4064) (layer "F.Cu") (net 23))
 (segment (start 124.46 90.17) (end 127 90.17) (width 0.4064) (layer "F.Cu") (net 24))
 (segment (start 124.46 92.71) (end 127 92.71) (width 0.4064) (layer "F.Cu") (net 25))
 (segment (start 124.46 97.79) (end 125.73 99.06) (width 0.3048) (layer "F.Cu") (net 27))
 (segment (start 129.54 85.13) (end 129.54 85.598) (width 0.3048) (layer "F.Cu") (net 27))
 (segment (start 129.54 85.598) (end 129.54 85.09) (width 0.3048) (layer "F.Cu") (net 27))
 (segment (start 133.985 80.685) (end 129.54 85.13) (width 0.3048) (layer "F.Cu") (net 27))
 (segment (start 129.54 97.155) (end 129.54 85.598) (width 0.3048) (layer "F.Cu") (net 27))
 (segment (start 127.635 99.06) (end 128.905 97.79) (width 0.3048) (layer "F.Cu") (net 27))
 (segment (start 128.905 97.79) (end 129.54 97.155) (width 0.3048) (layer "F.Cu") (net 27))
 (segment (start 125.73 99.06) (end 127.635 99.06) (width 0.3048) (layer "F.Cu") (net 27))
 (segment (start 128.27 100.33) (end 124.46 100.33) (width 0.3048) (layer "F.Cu") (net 15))
 (segment (start 137.16 97.028) (end 136.398 97.79) (width 0.3048) (layer "F.Cu") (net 15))
 (segment (start 137.16 93.345) (end 137.16 97.028) (width 0.3048) (layer "F.Cu") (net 15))
 (via (at 136.398 97.79) (size 0.6858) (drill 0.3302) (layers "F.Cu" "B.Cu") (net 15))
 (via (at 128.27 100.33) (size 0.6858) (drill 0.3302) (layers "F.Cu" "B.Cu") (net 15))
 (segment (start 128.27 100.33) (end 129.794 98.806) (width 0.3048) (layer "B.Cu") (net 15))
 (segment (start 129.794 98.806) (end 135.382 98.806) (width 0.3048) (layer "B.Cu") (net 15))
 (segment (start 135.382 98.806) (end 136.398 97.79) (width 0.3048) (layer "B.Cu") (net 15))
 (segment (start 130.445 100.33) (end 130.735 100.62) (width 0.3048) (layer "F.Cu") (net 17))
 (segment (start 125.476 101.854) (end 129.501 101.854) (width 0.3048) (layer "F.Cu") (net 17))
 (segment (start 129.501 101.854) (end 130.735 100.62) (width 0.3048) (layer "F.Cu") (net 17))
 (segment (start 124.46 102.87) (end 125.476 101.854) (width 0.3048) (layer "F.Cu") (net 17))
 (segment (start 130.735 100.62) (end 137.235 100.62) (width 0.4064) (layer "B.Cu") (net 17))
 (segment (start 132.08 109.93842) (end 132.08 111.76) (width 0.3048) (layer "F.Cu") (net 8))
 (segment (start 127.55158 105.41) (end 132.08 109.93842) (width 0.3048) (layer "F.Cu") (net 8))
 (segment (start 124.46 105.41) (end 127.55158 105.41) (width 0.3048) (layer "F.Cu") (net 8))
 (segment (start 124.46 113.03) (end 125.6765 113.03) (width 0.4064) (layer "F.Cu") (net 19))
 (segment (start 125.6765 113.03) (end 127 111.7065) (width 0.4064) (layer "F.Cu") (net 19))
 (segment (start 125.6765 115.57) (end 127 114.2465) (width 0.4064) (layer "F.Cu") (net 20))
 (segment (start 124.46 115.57) (end 125.6765 115.57) (width 0.4064) (layer "F.Cu") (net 20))
 (segment (start 124.46 118.11) (end 125.6765 118.11) (width 0.4064) (layer "F.Cu") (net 21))
 (segment (start 125.6765 118.11) (end 127 116.7865) (width 0.4064) (layer "F.Cu") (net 21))
 (segment (start 143.6878 121.7422) (end 143.6878 107.3658) (width 0.3048) (layer "F.Cu") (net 12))
 (segment (start 142.24 123.19) (end 143.6878 121.7422) (width 0.3048) (layer "F.Cu") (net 12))
 (segment (start 143.6878 107.3658) (end 143.002 106.68) (width 0.3048) (layer "F.Cu") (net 12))
 (segment (start 139.065 106.68) (end 136.525 109.22) (width 0.3048) (layer "F.Cu") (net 12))
 (segment (start 143.002 106.68) (end 139.065 106.68) (width 0.3048) (layer "F.Cu") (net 12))
 (segment (start 139.7 102.87) (end 142.24 105.41) (width 0.3048) (layer "B.Cu") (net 14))
 (segment (start 141.605 99.695) (end 142.24 100.33) (width 0.3048) (layer "B.Cu") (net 13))
 (segment (start 139.7 99.695) (end 141.605 99.695) (width 0.3048) (layer "B.Cu") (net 13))
 (segment (start 139.55 125.73) (end 140.82 124.46) (width 0.3048) (layer "F.Cu") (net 11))
 (segment (start 140.82 124.46) (end 142.875 124.46) (width 0.3048) (layer "F.Cu") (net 11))
 (segment (start 144.145 123.19) (end 144.145 99.695) (width 0.3048) (layer "F.Cu") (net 11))
 (segment (start 138.915 125.095) (end 139.55 125.73) (width 0.3048) (layer "F.Cu") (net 11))
 (segment (start 142.875 124.46) (end 144.145 123.19) (width 0.3048) (layer "F.Cu") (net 11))
 (segment (start 144.145 99.695) (end 142.24 97.79) (width 0.3048) (layer "F.Cu") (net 11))
 (segment (start 136.525 125.095) (end 138.915 125.095) (width 0.3048) (layer "F.Cu") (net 11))
 (segment (start 137.16 78.105) (end 139.065 80.01) (width 0.3048) (layer "B.Cu") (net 10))
 (segment (start 139.7 95.25) (end 136.398 95.25) (width 0.3048) (layer "B.Cu") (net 10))
 (segment (start 135.636 94.488) (end 135.636 82.169) (width 0.3048) (layer "B.Cu") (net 10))
 (segment (start 139.065 80.01) (end 139.7 80.01) (width 0.3048) (layer "B.Cu") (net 10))
 (segment (start 137.16 78.105) (end 137.16 80.645) (width 0.3048) (layer "B.Cu") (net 10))
 (segment (start 136.398 95.25) (end 135.636 94.488) (width 0.3048) (layer "B.Cu") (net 10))
 (segment (start 135.636 82.169) (end 135.89 81.915) (width 0.3048) (layer "B.Cu") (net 10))
 (segment (start 137.16 80.645) (end 135.89 81.915) (width 0.3048) (layer "B.Cu") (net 10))
 (segment (start 142.24 92.71) (end 139.7 95.25) (width 0.3048) (layer "B.Cu") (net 10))
 (segment (start 127 104.14) (end 128.27 102.87) (width 0.4064) (layer "F.Cu") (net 9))
 (segment (start 133.35 114.3) (end 134.3152 113.3348) (width 0.4064) (layer "F.Cu") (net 9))
 (segment (start 132.08 102.87) (end 133.35 101.6) (width 0.4064) (layer "F.Cu") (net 9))
 (segment (start 132.588 86.614) (end 135.128 89.154) (width 0.4064) (layer "F.Cu") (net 9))
 (segment (start 132.588 85.09) (end 132.588 86.614) (width 0.4064) (layer "F.Cu") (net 9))
 (segment (start 133.604 95.25) (end 133.35 95.25) (width 0.4064) (layer "F.Cu") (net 9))
 (segment (start 134.3152 113.3348) (end 134.3152 108.9152) (width 0.4064) (layer "F.Cu") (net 9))
 (segment (start 133.35 107.95) (end 130.81 107.95) (width 0.4064) (layer "F.Cu") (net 9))
 (segment (start 135.128 93.726) (end 133.604 95.25) (width 0.4064) (layer "F.Cu") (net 9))
 (segment (start 130.81 107.95) (end 127 104.14) (width 0.4064) (layer "F.Cu") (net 9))
 (segment (start 135.128 89.154) (end 135.128 93.726) (width 0.4064) (layer "F.Cu") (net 9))
 (segment (start 142.24 80.01) (end 141.0462 78.8162) (width 0.4064) (layer "F.Cu") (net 9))
 (segment (start 133.35 101.6) (end 133.35 95.25) (width 0.4064) (layer "F.Cu") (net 9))
 (segment (start 141.0462 78.8162) (end 138.8618 78.8162) (width 0.4064) (layer "F.Cu") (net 9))
 (segment (start 128.27 102.87) (end 132.08 102.87) (width 0.4064) (layer "F.Cu") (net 9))
 (segment (start 134.3152 108.9152) (end 133.35 107.95) (width 0.4064) (layer "F.Cu") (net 9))
 (segment (start 132.08 114.3) (end 133.35 114.3) (width 0.4064) (layer "F.Cu") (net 9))
 (segment (start 138.8618 78.8162) (end 132.588 85.09) (width 0.4064) (layer "F.Cu") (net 9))
 (segment (start 127 95.25) (end 133.35 95.25) (width 0.4064) (layer "B.Cu") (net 9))
 (segment (start 129.605 121.44) (end 128.425 121.44) (width 0.4064) (layer "B.Cu") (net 6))
 (segment (start 128.425 121.44) (end 125.7944 118.8094) (width 0.4064) (layer "B.Cu") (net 6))
 (segment (start 125.7944 118.8094) (end 125.7944 83.7556) (width 0.4064) (layer "B.Cu") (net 6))
 (segment (start 127.79 81.76) (end 129.54 81.76) (width 0.4064) (layer "B.Cu") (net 6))
 (segment (start 125.7944 83.7556) (end 127.79 81.76) (width 0.4064) (layer "B.Cu") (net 6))
 (segment (start 129.54 78.26) (end 129.695 78.26) (width 0.4064) (layer "B.Cu") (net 7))
 (segment (start 131.445 80.01) (end 131.445 90.805) (width 0.4064) (layer "B.Cu") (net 7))
 (segment (start 131.445 90.805) (end 133.35 92.71) (width 0.4064) (layer "B.Cu") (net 7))
 (segment (start 129.695 78.26) (end 131.445 80.01) (width 0.4064) (layer "B.Cu") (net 7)))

